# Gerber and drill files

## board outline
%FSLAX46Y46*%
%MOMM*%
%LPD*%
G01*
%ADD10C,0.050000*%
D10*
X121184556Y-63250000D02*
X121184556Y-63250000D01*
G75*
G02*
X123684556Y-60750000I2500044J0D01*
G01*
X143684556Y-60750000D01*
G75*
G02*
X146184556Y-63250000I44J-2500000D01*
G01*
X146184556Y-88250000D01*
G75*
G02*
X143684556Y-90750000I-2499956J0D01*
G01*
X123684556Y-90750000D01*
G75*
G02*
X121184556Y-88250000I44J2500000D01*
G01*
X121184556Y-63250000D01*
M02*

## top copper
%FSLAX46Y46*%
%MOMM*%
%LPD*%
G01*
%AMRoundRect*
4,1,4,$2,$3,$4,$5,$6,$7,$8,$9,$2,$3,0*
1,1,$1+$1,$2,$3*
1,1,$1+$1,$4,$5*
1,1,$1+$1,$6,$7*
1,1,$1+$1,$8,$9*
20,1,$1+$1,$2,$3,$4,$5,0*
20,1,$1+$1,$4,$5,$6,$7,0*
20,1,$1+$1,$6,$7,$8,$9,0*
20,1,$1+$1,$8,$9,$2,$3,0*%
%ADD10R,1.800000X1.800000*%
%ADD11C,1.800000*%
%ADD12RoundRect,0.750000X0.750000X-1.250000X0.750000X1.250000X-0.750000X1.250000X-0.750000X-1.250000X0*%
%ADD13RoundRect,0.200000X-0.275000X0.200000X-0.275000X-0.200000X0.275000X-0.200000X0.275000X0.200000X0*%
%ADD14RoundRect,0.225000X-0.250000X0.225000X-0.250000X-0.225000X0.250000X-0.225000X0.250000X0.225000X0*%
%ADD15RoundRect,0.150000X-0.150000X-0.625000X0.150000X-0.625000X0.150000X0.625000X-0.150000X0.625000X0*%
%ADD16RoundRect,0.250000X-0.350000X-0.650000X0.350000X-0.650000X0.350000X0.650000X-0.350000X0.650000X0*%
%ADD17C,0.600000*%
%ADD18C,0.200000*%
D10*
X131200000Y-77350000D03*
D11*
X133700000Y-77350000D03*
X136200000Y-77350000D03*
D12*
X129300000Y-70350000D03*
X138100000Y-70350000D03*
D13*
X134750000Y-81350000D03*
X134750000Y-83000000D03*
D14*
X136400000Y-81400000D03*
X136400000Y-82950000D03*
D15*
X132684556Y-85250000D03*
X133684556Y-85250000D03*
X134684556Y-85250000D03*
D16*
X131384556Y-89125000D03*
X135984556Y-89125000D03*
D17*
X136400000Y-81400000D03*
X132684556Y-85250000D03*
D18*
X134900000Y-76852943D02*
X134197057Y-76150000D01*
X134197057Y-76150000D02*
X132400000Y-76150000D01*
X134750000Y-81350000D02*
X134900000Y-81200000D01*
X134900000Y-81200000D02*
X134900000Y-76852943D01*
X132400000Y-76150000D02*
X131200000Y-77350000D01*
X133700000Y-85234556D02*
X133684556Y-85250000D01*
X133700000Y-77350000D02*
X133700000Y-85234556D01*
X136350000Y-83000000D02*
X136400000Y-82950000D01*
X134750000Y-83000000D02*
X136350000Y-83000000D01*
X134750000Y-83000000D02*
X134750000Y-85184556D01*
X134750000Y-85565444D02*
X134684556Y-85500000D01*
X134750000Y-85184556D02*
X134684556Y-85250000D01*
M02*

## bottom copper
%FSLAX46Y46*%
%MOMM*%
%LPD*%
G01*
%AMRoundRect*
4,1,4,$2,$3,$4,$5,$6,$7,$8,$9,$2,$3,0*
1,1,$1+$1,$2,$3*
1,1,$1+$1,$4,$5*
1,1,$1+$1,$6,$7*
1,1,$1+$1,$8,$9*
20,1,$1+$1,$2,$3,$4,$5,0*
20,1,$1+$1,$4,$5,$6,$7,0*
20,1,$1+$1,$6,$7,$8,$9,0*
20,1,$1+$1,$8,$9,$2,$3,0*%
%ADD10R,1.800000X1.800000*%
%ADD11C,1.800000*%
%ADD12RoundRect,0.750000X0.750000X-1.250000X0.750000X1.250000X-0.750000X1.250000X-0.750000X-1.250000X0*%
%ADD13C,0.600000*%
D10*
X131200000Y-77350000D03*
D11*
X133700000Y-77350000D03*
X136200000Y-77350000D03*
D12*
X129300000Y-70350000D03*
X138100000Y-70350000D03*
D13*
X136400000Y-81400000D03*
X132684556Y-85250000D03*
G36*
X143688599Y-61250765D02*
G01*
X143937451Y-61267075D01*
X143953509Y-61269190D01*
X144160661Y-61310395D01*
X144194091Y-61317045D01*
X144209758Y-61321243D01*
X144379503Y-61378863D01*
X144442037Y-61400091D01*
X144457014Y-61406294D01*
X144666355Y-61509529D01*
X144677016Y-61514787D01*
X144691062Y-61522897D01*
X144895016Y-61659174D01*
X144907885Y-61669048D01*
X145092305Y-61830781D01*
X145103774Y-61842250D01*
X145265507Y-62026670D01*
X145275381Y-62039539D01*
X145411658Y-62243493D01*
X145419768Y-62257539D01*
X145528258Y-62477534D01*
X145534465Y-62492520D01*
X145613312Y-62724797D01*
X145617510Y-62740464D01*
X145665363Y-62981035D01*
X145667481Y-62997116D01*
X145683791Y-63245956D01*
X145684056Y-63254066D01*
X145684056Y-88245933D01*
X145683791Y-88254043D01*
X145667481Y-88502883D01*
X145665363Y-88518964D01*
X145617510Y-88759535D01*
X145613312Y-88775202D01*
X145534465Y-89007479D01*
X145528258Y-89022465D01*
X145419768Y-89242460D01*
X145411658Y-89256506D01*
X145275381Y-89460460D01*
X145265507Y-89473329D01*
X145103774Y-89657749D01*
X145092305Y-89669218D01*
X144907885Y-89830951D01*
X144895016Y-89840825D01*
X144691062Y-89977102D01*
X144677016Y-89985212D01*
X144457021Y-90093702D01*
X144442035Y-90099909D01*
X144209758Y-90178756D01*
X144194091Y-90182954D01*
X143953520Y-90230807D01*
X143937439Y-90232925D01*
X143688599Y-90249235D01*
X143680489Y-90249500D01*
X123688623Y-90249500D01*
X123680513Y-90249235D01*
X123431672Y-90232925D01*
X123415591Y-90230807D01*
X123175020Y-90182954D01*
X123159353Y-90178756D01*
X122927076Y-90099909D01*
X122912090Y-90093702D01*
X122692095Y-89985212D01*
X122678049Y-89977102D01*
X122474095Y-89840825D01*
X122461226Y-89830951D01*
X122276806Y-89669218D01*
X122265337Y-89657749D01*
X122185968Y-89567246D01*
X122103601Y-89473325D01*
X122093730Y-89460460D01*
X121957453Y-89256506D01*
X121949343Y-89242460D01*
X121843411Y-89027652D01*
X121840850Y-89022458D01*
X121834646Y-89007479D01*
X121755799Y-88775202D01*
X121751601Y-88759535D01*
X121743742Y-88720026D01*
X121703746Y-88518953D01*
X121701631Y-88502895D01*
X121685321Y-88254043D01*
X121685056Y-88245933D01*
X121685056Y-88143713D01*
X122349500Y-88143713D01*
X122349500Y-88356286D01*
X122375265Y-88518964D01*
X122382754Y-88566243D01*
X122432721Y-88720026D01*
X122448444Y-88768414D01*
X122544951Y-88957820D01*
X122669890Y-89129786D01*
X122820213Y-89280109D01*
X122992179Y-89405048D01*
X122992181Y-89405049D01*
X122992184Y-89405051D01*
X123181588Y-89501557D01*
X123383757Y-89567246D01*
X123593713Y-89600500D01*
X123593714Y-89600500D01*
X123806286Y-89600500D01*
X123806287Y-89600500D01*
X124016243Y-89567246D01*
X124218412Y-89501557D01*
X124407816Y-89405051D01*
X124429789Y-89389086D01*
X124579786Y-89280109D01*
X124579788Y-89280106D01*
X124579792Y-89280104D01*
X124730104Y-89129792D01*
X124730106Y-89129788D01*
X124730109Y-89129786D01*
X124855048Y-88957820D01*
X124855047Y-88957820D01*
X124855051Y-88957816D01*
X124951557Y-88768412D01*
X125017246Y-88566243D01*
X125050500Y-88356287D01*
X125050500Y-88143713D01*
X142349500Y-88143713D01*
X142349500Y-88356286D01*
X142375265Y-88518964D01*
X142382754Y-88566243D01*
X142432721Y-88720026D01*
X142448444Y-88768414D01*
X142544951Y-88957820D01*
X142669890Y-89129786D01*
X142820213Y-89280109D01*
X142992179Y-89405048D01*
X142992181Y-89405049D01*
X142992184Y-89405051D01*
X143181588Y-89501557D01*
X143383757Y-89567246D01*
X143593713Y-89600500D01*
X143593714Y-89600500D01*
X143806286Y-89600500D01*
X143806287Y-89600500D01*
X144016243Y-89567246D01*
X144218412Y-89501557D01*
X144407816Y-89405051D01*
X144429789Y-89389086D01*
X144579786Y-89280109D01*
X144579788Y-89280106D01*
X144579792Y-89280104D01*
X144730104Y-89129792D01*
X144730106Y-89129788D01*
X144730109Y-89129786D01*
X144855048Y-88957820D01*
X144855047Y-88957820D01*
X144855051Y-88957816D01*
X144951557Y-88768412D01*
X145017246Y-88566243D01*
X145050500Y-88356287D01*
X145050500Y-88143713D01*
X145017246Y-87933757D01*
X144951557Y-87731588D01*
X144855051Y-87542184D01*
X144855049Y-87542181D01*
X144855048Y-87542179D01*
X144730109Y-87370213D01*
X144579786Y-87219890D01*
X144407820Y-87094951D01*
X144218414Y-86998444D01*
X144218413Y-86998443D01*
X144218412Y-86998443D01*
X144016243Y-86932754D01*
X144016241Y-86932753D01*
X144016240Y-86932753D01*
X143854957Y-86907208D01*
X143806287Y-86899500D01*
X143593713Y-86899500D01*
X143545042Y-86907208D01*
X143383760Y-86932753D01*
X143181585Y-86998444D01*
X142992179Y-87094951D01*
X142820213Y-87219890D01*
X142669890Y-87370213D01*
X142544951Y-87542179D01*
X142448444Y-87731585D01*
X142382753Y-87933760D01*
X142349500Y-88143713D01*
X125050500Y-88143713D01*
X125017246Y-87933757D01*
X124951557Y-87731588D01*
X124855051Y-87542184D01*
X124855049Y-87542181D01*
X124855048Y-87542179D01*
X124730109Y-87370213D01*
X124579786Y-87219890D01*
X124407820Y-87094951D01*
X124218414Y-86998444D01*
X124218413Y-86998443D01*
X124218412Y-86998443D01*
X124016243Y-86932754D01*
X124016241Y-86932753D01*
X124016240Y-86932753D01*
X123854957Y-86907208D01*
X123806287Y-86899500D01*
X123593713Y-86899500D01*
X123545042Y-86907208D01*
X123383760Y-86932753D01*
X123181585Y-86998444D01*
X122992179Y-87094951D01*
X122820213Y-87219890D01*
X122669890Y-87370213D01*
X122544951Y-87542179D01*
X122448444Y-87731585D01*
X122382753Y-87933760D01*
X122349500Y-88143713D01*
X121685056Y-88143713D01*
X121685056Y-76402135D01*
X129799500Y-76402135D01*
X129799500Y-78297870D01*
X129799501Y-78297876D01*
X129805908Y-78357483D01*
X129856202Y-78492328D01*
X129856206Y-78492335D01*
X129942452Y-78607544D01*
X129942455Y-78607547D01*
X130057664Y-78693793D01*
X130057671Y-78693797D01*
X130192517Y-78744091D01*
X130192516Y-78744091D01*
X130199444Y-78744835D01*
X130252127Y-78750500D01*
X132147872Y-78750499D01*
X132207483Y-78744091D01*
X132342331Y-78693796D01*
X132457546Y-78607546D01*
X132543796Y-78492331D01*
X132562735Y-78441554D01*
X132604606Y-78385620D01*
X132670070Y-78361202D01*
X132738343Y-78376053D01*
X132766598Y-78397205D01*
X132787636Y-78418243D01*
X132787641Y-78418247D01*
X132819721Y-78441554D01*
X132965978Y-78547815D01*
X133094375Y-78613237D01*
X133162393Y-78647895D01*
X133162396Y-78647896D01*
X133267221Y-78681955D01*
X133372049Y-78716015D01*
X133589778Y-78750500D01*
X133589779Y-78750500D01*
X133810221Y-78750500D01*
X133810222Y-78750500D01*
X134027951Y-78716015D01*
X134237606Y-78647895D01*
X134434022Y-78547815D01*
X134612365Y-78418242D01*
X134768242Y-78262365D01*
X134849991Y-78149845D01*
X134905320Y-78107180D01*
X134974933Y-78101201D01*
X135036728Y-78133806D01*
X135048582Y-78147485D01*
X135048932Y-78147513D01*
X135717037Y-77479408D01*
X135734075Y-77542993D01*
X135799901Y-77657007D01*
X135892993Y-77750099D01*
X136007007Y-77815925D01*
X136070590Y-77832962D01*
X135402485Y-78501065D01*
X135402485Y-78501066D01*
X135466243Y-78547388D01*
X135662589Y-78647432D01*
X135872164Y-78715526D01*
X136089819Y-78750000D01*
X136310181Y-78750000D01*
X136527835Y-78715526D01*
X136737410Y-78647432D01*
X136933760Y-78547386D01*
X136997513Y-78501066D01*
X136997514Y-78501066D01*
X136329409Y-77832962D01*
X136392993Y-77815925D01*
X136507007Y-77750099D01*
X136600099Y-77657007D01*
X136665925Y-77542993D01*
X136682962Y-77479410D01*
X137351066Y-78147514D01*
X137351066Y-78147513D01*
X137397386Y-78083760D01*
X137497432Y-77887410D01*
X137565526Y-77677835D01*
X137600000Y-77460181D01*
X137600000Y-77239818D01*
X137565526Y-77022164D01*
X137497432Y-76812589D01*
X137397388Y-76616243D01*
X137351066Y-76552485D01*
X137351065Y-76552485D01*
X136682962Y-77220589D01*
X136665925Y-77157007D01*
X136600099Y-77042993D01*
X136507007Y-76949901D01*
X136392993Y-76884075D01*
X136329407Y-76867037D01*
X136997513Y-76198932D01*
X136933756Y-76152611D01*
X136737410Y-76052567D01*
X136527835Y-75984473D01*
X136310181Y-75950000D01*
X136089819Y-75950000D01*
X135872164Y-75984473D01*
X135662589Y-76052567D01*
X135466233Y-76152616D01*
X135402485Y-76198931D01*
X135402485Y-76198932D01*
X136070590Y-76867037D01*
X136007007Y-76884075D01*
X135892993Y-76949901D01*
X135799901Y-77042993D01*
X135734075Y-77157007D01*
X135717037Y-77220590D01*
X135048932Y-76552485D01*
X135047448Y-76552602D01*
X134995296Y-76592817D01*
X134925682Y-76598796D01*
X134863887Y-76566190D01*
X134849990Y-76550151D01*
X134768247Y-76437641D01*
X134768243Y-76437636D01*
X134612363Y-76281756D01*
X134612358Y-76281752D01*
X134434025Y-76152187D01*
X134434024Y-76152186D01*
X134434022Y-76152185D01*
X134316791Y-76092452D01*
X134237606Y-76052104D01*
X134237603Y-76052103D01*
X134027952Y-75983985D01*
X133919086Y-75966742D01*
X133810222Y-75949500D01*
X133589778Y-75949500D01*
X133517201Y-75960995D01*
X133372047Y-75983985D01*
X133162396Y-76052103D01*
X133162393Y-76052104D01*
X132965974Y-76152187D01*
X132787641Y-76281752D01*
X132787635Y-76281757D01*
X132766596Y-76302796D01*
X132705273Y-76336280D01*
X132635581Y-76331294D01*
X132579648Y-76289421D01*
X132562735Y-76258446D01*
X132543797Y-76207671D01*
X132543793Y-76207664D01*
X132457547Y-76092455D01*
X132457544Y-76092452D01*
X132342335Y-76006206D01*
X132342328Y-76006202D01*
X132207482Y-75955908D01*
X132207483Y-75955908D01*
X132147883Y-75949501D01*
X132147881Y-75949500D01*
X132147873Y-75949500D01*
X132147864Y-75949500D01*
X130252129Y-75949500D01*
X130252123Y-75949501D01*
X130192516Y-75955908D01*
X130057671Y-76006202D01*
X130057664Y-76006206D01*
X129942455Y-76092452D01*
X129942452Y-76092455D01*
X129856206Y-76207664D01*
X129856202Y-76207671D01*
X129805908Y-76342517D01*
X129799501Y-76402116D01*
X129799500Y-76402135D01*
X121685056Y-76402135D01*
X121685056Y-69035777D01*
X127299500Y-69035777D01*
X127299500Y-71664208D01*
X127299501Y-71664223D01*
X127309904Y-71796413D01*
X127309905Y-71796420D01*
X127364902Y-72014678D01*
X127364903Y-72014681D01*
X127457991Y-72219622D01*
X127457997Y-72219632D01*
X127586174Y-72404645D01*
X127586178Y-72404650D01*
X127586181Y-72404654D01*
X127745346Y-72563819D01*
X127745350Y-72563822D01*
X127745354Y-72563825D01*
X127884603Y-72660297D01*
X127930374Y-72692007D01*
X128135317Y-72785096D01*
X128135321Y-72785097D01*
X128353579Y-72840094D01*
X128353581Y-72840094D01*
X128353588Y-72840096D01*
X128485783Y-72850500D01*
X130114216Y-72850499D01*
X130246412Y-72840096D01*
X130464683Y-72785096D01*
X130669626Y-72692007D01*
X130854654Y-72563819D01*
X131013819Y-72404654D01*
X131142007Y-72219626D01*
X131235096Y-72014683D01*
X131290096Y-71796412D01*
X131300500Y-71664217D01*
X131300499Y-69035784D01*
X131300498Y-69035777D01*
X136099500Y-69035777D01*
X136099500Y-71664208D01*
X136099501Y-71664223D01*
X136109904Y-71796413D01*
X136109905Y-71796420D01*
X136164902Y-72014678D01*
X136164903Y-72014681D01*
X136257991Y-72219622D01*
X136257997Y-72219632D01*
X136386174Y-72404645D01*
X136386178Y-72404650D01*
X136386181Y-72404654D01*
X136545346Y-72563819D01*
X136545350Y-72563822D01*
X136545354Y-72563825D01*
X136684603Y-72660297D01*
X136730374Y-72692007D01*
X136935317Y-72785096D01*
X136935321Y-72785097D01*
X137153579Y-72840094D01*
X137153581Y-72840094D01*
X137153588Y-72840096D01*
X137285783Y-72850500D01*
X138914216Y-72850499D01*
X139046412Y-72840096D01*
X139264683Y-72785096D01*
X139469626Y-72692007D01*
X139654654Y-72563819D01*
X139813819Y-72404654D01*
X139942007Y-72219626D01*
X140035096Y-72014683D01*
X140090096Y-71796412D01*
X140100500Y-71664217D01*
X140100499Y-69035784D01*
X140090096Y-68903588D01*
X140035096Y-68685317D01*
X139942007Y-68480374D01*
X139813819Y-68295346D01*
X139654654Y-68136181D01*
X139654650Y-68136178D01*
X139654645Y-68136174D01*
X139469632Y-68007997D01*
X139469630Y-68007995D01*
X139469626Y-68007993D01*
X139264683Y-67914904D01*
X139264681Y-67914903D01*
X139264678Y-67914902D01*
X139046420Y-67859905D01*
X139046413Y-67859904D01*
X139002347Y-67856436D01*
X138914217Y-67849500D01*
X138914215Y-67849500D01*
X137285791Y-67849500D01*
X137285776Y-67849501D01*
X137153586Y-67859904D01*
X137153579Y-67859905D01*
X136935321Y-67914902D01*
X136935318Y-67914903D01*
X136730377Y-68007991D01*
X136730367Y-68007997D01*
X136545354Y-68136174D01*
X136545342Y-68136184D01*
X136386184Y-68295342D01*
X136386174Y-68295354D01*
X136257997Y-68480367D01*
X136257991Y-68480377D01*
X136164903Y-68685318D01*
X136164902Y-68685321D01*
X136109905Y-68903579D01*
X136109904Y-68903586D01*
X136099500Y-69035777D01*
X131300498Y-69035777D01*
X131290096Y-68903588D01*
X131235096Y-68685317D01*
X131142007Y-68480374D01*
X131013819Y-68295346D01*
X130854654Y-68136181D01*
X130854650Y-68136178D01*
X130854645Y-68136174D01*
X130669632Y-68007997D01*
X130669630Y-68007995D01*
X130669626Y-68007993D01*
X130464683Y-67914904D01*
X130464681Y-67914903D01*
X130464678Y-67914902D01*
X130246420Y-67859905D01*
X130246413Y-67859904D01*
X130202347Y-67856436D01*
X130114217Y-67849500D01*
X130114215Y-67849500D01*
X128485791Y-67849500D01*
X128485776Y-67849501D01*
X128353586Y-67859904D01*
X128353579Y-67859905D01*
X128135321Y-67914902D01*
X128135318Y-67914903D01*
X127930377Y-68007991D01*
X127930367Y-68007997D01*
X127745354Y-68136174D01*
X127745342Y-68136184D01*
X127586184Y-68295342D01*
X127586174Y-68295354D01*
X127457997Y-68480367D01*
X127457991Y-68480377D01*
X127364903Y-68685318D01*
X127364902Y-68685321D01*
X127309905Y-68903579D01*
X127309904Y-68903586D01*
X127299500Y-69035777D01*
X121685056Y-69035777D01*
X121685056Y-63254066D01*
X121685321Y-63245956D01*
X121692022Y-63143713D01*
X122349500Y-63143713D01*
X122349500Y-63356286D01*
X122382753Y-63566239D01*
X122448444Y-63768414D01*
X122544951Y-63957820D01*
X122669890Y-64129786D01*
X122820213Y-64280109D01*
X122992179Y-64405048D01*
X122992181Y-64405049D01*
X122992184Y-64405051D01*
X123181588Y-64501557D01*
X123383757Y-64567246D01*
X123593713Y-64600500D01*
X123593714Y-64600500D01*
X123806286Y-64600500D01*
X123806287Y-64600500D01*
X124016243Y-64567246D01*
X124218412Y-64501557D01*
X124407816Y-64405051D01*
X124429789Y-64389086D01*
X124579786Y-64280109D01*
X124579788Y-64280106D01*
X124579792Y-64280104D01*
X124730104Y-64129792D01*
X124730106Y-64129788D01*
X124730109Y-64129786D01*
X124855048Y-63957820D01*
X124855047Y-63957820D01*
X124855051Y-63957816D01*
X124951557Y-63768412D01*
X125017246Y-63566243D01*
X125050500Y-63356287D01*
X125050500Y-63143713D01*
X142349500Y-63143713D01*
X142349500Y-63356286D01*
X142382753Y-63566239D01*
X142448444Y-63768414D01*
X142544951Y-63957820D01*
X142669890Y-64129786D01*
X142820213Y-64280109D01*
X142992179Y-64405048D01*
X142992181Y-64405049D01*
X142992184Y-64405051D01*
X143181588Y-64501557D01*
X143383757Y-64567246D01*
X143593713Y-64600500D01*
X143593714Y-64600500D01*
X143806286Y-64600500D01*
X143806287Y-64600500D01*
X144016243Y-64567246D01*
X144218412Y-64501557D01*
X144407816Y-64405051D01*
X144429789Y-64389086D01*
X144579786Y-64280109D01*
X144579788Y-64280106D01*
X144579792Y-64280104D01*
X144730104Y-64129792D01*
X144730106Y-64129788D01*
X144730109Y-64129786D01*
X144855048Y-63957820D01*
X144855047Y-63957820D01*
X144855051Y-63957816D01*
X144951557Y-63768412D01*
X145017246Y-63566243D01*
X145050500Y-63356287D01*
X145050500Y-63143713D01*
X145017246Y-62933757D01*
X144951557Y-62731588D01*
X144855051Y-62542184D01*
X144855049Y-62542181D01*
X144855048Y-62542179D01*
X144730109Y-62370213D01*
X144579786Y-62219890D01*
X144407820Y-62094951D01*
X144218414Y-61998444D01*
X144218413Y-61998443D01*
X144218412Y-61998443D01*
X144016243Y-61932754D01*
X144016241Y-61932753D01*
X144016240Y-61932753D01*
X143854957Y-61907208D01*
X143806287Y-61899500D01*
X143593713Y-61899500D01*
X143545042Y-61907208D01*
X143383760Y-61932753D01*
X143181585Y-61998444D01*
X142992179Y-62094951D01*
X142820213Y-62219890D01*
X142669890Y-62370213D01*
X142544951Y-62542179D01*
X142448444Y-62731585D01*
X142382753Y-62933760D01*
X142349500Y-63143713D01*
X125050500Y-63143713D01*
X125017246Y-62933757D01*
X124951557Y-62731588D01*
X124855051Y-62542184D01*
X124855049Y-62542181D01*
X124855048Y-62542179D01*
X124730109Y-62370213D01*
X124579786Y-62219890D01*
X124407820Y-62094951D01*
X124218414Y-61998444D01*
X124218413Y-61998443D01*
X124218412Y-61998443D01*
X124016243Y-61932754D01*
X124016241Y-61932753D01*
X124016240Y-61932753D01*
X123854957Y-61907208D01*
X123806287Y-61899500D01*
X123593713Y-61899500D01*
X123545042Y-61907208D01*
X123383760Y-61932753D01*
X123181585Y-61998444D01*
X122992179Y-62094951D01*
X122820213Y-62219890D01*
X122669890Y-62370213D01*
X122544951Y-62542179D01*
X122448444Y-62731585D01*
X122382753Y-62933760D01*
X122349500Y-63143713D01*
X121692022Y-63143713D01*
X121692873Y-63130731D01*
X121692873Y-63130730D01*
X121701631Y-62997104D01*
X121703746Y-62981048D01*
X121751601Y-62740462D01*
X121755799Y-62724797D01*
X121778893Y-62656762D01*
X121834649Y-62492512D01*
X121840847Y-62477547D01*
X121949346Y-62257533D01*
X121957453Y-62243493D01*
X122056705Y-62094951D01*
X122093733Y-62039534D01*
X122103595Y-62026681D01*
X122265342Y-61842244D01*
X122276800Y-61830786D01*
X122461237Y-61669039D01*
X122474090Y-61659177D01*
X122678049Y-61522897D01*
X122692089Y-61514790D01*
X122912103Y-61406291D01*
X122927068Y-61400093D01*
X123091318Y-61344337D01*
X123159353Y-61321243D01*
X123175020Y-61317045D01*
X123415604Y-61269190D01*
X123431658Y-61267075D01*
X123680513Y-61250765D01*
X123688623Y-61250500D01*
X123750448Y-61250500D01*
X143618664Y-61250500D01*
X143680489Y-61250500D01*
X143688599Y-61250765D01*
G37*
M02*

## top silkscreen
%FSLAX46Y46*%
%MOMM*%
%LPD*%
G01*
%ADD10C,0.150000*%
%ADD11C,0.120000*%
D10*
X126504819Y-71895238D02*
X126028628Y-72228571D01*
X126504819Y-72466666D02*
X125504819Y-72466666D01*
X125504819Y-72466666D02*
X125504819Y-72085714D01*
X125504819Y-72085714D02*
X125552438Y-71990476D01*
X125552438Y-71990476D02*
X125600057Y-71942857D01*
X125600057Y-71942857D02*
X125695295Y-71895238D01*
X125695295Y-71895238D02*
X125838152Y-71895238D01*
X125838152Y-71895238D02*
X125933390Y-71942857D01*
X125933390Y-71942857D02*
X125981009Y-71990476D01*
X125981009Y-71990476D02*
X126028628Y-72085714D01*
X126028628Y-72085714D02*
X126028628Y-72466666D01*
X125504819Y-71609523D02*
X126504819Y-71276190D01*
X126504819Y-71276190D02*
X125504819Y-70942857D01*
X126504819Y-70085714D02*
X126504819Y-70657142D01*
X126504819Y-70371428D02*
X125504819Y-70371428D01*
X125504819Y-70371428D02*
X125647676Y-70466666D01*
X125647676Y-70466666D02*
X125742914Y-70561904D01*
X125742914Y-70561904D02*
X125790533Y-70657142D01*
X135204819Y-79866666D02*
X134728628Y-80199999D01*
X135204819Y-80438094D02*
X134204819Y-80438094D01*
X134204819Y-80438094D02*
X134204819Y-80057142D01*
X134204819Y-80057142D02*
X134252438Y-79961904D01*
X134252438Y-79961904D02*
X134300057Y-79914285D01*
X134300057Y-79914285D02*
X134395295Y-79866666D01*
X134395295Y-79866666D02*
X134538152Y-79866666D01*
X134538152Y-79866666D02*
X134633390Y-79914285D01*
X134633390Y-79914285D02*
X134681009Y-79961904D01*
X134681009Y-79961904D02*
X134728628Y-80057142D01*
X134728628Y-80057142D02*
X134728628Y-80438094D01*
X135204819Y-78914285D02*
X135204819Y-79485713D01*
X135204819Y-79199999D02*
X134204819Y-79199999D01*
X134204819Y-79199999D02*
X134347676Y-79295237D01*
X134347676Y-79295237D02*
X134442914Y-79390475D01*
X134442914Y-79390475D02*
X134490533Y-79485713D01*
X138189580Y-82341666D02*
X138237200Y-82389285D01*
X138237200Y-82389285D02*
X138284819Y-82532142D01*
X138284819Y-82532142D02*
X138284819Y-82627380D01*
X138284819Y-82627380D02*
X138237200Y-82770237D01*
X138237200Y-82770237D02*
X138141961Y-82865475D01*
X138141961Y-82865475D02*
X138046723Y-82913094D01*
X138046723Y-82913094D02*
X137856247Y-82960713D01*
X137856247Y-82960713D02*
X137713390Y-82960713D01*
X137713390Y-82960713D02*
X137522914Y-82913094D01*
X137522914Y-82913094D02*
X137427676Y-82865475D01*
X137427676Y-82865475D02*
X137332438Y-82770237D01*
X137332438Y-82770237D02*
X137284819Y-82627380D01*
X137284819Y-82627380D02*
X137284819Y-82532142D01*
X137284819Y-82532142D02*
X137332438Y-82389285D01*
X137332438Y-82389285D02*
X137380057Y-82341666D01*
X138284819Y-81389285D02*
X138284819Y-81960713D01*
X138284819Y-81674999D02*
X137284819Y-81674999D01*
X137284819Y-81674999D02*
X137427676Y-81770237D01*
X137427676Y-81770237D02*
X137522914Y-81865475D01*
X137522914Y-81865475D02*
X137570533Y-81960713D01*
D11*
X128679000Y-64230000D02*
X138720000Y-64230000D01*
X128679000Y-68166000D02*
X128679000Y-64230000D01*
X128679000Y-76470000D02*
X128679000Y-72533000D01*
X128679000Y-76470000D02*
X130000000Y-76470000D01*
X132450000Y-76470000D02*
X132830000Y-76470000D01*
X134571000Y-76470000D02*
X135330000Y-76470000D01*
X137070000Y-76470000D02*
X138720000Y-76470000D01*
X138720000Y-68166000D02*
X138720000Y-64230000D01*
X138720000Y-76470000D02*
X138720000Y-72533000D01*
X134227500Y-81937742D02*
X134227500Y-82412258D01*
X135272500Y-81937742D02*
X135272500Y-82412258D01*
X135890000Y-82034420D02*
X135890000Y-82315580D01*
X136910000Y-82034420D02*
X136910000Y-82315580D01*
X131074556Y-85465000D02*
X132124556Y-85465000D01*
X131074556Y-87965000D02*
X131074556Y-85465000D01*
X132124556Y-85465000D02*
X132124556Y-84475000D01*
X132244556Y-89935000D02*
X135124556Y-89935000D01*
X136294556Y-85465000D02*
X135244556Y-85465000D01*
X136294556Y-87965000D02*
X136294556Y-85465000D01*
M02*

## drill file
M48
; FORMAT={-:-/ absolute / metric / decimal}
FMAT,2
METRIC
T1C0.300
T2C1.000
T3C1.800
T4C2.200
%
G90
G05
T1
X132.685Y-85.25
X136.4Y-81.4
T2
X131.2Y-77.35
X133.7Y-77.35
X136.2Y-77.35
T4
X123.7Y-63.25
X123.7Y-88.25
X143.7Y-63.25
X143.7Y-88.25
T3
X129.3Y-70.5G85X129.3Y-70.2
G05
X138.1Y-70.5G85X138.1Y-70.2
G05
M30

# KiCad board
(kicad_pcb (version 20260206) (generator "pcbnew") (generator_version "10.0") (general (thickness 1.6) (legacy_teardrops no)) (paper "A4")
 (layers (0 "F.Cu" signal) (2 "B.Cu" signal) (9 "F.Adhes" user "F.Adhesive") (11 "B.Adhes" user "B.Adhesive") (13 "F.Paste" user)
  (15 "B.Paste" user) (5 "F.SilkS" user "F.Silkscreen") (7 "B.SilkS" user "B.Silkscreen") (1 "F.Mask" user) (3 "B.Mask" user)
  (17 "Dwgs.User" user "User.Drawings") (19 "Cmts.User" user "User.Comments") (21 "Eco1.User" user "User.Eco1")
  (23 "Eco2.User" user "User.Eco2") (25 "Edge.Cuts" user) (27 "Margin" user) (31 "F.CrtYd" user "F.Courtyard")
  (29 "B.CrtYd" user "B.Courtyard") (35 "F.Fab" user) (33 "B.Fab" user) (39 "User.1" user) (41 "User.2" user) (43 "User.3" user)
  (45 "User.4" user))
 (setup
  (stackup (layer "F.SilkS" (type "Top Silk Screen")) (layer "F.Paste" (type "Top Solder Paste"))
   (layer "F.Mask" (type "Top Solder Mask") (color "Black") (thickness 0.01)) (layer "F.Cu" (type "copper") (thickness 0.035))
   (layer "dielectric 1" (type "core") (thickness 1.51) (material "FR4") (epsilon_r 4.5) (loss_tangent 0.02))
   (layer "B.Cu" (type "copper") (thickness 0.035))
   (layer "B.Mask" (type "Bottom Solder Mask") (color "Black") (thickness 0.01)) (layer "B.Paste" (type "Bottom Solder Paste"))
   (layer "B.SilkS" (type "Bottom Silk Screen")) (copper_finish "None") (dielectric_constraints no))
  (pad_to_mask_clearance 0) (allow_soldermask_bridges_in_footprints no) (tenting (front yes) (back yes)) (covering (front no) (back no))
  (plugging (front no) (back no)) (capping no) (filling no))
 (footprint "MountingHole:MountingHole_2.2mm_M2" (layer "F.Cu") (at 123.7 88.25)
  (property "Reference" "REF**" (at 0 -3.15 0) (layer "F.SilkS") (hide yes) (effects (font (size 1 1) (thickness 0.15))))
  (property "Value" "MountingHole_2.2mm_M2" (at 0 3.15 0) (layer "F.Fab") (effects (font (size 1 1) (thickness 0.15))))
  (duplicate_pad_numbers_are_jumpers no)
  (pad "" np_thru_hole circle (at 0 0) (size 2.2 2.2) (drill 2.2) (layers "*.Cu" "*.Mask")))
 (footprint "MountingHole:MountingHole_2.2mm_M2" (layer "F.Cu") (at 143.7 63.25)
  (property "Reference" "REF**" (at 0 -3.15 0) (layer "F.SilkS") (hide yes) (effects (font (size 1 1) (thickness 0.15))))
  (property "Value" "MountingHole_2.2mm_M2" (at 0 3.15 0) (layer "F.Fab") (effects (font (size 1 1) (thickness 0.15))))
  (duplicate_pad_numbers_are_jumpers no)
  (pad "" np_thru_hole circle (at 0 0) (size 2.2 2.2) (drill 2.2) (layers "*.Cu" "*.Mask")))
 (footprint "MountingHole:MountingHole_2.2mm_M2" (layer "F.Cu") (at 143.7 88.25)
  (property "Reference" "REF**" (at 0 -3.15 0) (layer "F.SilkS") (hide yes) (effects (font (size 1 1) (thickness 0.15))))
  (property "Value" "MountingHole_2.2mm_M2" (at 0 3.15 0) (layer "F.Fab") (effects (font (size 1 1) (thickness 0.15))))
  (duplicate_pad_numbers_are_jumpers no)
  (pad "" np_thru_hole circle (at 0 0) (size 2.2 2.2) (drill 2.2) (layers "*.Cu" "*.Mask")))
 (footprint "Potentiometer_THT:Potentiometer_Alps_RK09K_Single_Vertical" (layer "F.Cu") (at 131.2 77.35 90)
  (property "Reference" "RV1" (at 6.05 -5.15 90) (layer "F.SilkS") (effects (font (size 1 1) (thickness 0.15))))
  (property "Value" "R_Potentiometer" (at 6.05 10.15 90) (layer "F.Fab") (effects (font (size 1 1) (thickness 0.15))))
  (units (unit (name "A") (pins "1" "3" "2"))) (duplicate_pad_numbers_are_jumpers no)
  (fp_line (start 13.12 -2.521) (end 13.12 7.52) (stroke (width 0.12) (type solid)) (layer "F.SilkS"))
  (fp_line (start 9.184 -2.521) (end 13.12 -2.521) (stroke (width 0.12) (type solid)) (layer "F.SilkS"))
  (fp_line (start 0.88 -2.521) (end 4.817 -2.521) (stroke (width 0.12) (type solid)) (layer "F.SilkS"))
  (fp_line (start 0.88 -2.521) (end 0.88 -1.2) (stroke (width 0.12) (type solid)) (layer "F.SilkS"))
  (fp_line (start 0.88 1.25) (end 0.88 1.63) (stroke (width 0.12) (type solid)) (layer "F.SilkS"))
  (fp_line (start 0.88 3.371) (end 0.88 4.13) (stroke (width 0.12) (type solid)) (layer "F.SilkS"))
  (fp_line (start 0.88 5.87) (end 0.88 7.52) (stroke (width 0.12) (type solid)) (layer "F.SilkS"))
  (fp_line (start 9.184 7.52) (end 13.12 7.52) (stroke (width 0.12) (type solid)) (layer "F.SilkS"))
  (fp_line (start 0.88 7.52) (end 4.817 7.52) (stroke (width 0.12) (type solid)) (layer "F.SilkS"))
  (pad "1" thru_hole rect (at 0 0 90) (size 1.8 1.8) (drill 1) (layers "*.Cu" "*.Mask") (remove_unused_layers no) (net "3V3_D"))
  (pad "2" thru_hole circle (at 0 2.5 90) (size 1.8 1.8) (drill 1) (layers "*.Cu" "*.Mask") (remove_unused_layers no) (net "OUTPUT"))
  (pad "3" thru_hole circle (at 0 5 90) (size 1.8 1.8) (drill 1) (layers "*.Cu" "*.Mask") (remove_unused_layers no) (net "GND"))
  (pad "MP" thru_hole roundrect (at 7 -1.9 90) (size 4 3) (drill oval 2.1 1.8) (layers "*.Cu" "*.Mask") (remove_unused_layers no)
   (roundrect_rratio 0.25))
  (pad "MP" thru_hole roundrect (at 7 6.9 90) (size 4 3) (drill oval 2.1 1.8) (layers "*.Cu" "*.Mask") (remove_unused_layers no)
   (roundrect_rratio 0.25)))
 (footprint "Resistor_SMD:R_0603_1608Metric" (layer "F.Cu") (at 134.75 82.175 -90)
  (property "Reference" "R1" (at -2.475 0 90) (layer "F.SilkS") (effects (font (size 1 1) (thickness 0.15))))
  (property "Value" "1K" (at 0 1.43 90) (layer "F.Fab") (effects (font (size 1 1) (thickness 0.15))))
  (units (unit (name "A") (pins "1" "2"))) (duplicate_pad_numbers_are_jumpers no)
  (fp_line (start -0.237258 0.5225) (end 0.237258 0.5225) (stroke (width 0.12) (type solid)) (layer "F.SilkS"))
  (fp_line (start -0.237258 -0.5225) (end 0.237258 -0.5225) (stroke (width 0.12) (type solid)) (layer "F.SilkS"))
  (pad "1" smd roundrect (at -0.825 0 270) (size 0.8 0.95) (layers "F.Cu" "F.Mask" "F.Paste") (roundrect_rratio 0.25) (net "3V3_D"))
  (pad "2" smd roundrect (at 0.825 0 270) (size 0.8 0.95) (layers "F.Cu" "F.Mask" "F.Paste") (roundrect_rratio 0.25) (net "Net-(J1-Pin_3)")))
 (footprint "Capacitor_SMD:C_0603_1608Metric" (layer "F.Cu") (at 136.4 82.175 -90)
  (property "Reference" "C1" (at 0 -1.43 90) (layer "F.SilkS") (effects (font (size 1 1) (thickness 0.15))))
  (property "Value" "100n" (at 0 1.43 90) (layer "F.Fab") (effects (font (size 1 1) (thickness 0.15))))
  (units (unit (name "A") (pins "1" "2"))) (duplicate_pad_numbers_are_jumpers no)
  (fp_line (start -0.14058 0.51) (end 0.14058 0.51) (stroke (width 0.12) (type solid)) (layer "F.SilkS"))
  (fp_line (start -0.14058 -0.51) (end 0.14058 -0.51) (stroke (width 0.12) (type solid)) (layer "F.SilkS"))
  (pad "1" smd roundrect (at -0.775 0 270) (size 0.9 0.95) (layers "F.Cu" "F.Mask" "F.Paste") (roundrect_rratio 0.25) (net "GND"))
  (pad "2" smd roundrect (at 0.775 0 270) (size 0.9 0.95) (layers "F.Cu" "F.Mask" "F.Paste") (roundrect_rratio 0.25) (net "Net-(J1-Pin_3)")))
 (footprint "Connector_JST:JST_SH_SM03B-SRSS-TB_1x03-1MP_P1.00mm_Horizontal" (layer "F.Cu") (at 133.684556 87.25)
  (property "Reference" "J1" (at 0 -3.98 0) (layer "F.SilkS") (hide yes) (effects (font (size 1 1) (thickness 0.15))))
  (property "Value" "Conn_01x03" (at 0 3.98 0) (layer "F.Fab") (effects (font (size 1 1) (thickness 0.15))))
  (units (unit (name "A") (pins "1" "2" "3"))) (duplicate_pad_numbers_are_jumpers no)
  (fp_line (start -2.61 -1.785) (end -1.56 -1.785) (stroke (width 0.12) (type solid)) (layer "F.SilkS"))
  (fp_line (start -2.61 0.715) (end -2.61 -1.785) (stroke (width 0.12) (type solid)) (layer "F.SilkS"))
  (fp_line (start -1.56 -1.785) (end -1.56 -2.775) (stroke (width 0.12) (type solid)) (layer "F.SilkS"))
  (fp_line (start -1.44 2.685) (end 1.44 2.685) (stroke (width 0.12) (type solid)) (layer "F.SilkS"))
  (fp_line (start 2.61 -1.785) (end 1.56 -1.785) (stroke (width 0.12) (type solid)) (layer "F.SilkS"))
  (fp_line (start 2.61 0.715) (end 2.61 -1.785) (stroke (width 0.12) (type solid)) (layer "F.SilkS"))
  (pad "1" smd roundrect (at -1 -2) (size 0.6 1.55) (layers "F.Cu" "F.Mask" "F.Paste") (roundrect_rratio 0.25) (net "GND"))
  (pad "2" smd roundrect (at 0 -2) (size 0.6 1.55) (layers "F.Cu" "F.Mask" "F.Paste") (roundrect_rratio 0.25) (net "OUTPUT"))
  (pad "3" smd roundrect (at 1 -2) (size 0.6 1.55) (layers "F.Cu" "F.Mask" "F.Paste") (roundrect_rratio 0.25) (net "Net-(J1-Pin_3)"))
  (pad "MP" smd roundrect (at -2.3 1.875) (size 1.2 1.8) (layers "F.Cu" "F.Mask" "F.Paste") (roundrect_rratio 0.208333))
  (pad "MP" smd roundrect (at 2.3 1.875) (size 1.2 1.8) (layers "F.Cu" "F.Mask" "F.Paste") (roundrect_rratio 0.208333)))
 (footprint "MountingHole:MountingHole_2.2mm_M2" (layer "F.Cu") (at 123.7 63.25)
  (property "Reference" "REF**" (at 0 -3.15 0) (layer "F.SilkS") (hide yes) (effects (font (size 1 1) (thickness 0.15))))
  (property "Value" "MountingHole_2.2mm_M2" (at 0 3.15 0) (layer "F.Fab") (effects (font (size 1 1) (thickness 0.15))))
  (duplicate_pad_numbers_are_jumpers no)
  (pad "" np_thru_hole circle (at 0 0) (size 2.2 2.2) (drill 2.2) (layers "*.Cu" "*.Mask")))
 (gr_rect (start 121.184556 60.75) (end 146.184556 90.75) (radius 2.5) (stroke (width 0.05) (type solid)) (fill no) (layer "Edge.Cuts"))
 (segment (start 134.9 76.852943) (end 134.197057 76.15) (width 0.2) (layer "F.Cu") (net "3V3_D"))
 (segment (start 134.197057 76.15) (end 132.4 76.15) (width 0.2) (layer "F.Cu") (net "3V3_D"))
 (segment (start 134.75 81.35) (end 134.9 81.2) (width 0.2) (layer "F.Cu") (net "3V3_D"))
 (segment (start 134.9 81.2) (end 134.9 76.852943) (width 0.2) (layer "F.Cu") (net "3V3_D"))
 (segment (start 132.4 76.15) (end 131.2 77.35) (width 0.2) (layer "F.Cu") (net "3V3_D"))
 (segment (start 133.7 85.234556) (end 133.684556 85.25) (width 0.2) (layer "F.Cu") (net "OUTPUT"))
 (segment (start 133.7 77.35) (end 133.7 85.234556) (width 0.2) (layer "F.Cu") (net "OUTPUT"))
 (via (at 136.4 81.4) (size 0.6) (drill 0.3) (layers "F.Cu" "B.Cu") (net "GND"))
 (via (at 132.684556 85.25) (size 0.6) (drill 0.3) (layers "F.Cu" "B.Cu") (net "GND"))
 (segment (start 136.35 83) (end 136.4 82.95) (width 0.2) (layer "F.Cu") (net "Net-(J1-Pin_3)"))
 (segment (start 134.75 83) (end 136.35 83) (width 0.2) (layer "F.Cu") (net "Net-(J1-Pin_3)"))
 (segment (start 134.75 83) (end 134.75 85.184556) (width 0.2) (layer "F.Cu") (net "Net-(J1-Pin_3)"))
 (segment (start 134.75 85.565444) (end 134.684556 85.5) (width 0.2) (layer "F.Cu") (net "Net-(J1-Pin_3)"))
 (segment (start 134.75 85.184556) (end 134.684556 85.25) (width 0.2) (layer "F.Cu") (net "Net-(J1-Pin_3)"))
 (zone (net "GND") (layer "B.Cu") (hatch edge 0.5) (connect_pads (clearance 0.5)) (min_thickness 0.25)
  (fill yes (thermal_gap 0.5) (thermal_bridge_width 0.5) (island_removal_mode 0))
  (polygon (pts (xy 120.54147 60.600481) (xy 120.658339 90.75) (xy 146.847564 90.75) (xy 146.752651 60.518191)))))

